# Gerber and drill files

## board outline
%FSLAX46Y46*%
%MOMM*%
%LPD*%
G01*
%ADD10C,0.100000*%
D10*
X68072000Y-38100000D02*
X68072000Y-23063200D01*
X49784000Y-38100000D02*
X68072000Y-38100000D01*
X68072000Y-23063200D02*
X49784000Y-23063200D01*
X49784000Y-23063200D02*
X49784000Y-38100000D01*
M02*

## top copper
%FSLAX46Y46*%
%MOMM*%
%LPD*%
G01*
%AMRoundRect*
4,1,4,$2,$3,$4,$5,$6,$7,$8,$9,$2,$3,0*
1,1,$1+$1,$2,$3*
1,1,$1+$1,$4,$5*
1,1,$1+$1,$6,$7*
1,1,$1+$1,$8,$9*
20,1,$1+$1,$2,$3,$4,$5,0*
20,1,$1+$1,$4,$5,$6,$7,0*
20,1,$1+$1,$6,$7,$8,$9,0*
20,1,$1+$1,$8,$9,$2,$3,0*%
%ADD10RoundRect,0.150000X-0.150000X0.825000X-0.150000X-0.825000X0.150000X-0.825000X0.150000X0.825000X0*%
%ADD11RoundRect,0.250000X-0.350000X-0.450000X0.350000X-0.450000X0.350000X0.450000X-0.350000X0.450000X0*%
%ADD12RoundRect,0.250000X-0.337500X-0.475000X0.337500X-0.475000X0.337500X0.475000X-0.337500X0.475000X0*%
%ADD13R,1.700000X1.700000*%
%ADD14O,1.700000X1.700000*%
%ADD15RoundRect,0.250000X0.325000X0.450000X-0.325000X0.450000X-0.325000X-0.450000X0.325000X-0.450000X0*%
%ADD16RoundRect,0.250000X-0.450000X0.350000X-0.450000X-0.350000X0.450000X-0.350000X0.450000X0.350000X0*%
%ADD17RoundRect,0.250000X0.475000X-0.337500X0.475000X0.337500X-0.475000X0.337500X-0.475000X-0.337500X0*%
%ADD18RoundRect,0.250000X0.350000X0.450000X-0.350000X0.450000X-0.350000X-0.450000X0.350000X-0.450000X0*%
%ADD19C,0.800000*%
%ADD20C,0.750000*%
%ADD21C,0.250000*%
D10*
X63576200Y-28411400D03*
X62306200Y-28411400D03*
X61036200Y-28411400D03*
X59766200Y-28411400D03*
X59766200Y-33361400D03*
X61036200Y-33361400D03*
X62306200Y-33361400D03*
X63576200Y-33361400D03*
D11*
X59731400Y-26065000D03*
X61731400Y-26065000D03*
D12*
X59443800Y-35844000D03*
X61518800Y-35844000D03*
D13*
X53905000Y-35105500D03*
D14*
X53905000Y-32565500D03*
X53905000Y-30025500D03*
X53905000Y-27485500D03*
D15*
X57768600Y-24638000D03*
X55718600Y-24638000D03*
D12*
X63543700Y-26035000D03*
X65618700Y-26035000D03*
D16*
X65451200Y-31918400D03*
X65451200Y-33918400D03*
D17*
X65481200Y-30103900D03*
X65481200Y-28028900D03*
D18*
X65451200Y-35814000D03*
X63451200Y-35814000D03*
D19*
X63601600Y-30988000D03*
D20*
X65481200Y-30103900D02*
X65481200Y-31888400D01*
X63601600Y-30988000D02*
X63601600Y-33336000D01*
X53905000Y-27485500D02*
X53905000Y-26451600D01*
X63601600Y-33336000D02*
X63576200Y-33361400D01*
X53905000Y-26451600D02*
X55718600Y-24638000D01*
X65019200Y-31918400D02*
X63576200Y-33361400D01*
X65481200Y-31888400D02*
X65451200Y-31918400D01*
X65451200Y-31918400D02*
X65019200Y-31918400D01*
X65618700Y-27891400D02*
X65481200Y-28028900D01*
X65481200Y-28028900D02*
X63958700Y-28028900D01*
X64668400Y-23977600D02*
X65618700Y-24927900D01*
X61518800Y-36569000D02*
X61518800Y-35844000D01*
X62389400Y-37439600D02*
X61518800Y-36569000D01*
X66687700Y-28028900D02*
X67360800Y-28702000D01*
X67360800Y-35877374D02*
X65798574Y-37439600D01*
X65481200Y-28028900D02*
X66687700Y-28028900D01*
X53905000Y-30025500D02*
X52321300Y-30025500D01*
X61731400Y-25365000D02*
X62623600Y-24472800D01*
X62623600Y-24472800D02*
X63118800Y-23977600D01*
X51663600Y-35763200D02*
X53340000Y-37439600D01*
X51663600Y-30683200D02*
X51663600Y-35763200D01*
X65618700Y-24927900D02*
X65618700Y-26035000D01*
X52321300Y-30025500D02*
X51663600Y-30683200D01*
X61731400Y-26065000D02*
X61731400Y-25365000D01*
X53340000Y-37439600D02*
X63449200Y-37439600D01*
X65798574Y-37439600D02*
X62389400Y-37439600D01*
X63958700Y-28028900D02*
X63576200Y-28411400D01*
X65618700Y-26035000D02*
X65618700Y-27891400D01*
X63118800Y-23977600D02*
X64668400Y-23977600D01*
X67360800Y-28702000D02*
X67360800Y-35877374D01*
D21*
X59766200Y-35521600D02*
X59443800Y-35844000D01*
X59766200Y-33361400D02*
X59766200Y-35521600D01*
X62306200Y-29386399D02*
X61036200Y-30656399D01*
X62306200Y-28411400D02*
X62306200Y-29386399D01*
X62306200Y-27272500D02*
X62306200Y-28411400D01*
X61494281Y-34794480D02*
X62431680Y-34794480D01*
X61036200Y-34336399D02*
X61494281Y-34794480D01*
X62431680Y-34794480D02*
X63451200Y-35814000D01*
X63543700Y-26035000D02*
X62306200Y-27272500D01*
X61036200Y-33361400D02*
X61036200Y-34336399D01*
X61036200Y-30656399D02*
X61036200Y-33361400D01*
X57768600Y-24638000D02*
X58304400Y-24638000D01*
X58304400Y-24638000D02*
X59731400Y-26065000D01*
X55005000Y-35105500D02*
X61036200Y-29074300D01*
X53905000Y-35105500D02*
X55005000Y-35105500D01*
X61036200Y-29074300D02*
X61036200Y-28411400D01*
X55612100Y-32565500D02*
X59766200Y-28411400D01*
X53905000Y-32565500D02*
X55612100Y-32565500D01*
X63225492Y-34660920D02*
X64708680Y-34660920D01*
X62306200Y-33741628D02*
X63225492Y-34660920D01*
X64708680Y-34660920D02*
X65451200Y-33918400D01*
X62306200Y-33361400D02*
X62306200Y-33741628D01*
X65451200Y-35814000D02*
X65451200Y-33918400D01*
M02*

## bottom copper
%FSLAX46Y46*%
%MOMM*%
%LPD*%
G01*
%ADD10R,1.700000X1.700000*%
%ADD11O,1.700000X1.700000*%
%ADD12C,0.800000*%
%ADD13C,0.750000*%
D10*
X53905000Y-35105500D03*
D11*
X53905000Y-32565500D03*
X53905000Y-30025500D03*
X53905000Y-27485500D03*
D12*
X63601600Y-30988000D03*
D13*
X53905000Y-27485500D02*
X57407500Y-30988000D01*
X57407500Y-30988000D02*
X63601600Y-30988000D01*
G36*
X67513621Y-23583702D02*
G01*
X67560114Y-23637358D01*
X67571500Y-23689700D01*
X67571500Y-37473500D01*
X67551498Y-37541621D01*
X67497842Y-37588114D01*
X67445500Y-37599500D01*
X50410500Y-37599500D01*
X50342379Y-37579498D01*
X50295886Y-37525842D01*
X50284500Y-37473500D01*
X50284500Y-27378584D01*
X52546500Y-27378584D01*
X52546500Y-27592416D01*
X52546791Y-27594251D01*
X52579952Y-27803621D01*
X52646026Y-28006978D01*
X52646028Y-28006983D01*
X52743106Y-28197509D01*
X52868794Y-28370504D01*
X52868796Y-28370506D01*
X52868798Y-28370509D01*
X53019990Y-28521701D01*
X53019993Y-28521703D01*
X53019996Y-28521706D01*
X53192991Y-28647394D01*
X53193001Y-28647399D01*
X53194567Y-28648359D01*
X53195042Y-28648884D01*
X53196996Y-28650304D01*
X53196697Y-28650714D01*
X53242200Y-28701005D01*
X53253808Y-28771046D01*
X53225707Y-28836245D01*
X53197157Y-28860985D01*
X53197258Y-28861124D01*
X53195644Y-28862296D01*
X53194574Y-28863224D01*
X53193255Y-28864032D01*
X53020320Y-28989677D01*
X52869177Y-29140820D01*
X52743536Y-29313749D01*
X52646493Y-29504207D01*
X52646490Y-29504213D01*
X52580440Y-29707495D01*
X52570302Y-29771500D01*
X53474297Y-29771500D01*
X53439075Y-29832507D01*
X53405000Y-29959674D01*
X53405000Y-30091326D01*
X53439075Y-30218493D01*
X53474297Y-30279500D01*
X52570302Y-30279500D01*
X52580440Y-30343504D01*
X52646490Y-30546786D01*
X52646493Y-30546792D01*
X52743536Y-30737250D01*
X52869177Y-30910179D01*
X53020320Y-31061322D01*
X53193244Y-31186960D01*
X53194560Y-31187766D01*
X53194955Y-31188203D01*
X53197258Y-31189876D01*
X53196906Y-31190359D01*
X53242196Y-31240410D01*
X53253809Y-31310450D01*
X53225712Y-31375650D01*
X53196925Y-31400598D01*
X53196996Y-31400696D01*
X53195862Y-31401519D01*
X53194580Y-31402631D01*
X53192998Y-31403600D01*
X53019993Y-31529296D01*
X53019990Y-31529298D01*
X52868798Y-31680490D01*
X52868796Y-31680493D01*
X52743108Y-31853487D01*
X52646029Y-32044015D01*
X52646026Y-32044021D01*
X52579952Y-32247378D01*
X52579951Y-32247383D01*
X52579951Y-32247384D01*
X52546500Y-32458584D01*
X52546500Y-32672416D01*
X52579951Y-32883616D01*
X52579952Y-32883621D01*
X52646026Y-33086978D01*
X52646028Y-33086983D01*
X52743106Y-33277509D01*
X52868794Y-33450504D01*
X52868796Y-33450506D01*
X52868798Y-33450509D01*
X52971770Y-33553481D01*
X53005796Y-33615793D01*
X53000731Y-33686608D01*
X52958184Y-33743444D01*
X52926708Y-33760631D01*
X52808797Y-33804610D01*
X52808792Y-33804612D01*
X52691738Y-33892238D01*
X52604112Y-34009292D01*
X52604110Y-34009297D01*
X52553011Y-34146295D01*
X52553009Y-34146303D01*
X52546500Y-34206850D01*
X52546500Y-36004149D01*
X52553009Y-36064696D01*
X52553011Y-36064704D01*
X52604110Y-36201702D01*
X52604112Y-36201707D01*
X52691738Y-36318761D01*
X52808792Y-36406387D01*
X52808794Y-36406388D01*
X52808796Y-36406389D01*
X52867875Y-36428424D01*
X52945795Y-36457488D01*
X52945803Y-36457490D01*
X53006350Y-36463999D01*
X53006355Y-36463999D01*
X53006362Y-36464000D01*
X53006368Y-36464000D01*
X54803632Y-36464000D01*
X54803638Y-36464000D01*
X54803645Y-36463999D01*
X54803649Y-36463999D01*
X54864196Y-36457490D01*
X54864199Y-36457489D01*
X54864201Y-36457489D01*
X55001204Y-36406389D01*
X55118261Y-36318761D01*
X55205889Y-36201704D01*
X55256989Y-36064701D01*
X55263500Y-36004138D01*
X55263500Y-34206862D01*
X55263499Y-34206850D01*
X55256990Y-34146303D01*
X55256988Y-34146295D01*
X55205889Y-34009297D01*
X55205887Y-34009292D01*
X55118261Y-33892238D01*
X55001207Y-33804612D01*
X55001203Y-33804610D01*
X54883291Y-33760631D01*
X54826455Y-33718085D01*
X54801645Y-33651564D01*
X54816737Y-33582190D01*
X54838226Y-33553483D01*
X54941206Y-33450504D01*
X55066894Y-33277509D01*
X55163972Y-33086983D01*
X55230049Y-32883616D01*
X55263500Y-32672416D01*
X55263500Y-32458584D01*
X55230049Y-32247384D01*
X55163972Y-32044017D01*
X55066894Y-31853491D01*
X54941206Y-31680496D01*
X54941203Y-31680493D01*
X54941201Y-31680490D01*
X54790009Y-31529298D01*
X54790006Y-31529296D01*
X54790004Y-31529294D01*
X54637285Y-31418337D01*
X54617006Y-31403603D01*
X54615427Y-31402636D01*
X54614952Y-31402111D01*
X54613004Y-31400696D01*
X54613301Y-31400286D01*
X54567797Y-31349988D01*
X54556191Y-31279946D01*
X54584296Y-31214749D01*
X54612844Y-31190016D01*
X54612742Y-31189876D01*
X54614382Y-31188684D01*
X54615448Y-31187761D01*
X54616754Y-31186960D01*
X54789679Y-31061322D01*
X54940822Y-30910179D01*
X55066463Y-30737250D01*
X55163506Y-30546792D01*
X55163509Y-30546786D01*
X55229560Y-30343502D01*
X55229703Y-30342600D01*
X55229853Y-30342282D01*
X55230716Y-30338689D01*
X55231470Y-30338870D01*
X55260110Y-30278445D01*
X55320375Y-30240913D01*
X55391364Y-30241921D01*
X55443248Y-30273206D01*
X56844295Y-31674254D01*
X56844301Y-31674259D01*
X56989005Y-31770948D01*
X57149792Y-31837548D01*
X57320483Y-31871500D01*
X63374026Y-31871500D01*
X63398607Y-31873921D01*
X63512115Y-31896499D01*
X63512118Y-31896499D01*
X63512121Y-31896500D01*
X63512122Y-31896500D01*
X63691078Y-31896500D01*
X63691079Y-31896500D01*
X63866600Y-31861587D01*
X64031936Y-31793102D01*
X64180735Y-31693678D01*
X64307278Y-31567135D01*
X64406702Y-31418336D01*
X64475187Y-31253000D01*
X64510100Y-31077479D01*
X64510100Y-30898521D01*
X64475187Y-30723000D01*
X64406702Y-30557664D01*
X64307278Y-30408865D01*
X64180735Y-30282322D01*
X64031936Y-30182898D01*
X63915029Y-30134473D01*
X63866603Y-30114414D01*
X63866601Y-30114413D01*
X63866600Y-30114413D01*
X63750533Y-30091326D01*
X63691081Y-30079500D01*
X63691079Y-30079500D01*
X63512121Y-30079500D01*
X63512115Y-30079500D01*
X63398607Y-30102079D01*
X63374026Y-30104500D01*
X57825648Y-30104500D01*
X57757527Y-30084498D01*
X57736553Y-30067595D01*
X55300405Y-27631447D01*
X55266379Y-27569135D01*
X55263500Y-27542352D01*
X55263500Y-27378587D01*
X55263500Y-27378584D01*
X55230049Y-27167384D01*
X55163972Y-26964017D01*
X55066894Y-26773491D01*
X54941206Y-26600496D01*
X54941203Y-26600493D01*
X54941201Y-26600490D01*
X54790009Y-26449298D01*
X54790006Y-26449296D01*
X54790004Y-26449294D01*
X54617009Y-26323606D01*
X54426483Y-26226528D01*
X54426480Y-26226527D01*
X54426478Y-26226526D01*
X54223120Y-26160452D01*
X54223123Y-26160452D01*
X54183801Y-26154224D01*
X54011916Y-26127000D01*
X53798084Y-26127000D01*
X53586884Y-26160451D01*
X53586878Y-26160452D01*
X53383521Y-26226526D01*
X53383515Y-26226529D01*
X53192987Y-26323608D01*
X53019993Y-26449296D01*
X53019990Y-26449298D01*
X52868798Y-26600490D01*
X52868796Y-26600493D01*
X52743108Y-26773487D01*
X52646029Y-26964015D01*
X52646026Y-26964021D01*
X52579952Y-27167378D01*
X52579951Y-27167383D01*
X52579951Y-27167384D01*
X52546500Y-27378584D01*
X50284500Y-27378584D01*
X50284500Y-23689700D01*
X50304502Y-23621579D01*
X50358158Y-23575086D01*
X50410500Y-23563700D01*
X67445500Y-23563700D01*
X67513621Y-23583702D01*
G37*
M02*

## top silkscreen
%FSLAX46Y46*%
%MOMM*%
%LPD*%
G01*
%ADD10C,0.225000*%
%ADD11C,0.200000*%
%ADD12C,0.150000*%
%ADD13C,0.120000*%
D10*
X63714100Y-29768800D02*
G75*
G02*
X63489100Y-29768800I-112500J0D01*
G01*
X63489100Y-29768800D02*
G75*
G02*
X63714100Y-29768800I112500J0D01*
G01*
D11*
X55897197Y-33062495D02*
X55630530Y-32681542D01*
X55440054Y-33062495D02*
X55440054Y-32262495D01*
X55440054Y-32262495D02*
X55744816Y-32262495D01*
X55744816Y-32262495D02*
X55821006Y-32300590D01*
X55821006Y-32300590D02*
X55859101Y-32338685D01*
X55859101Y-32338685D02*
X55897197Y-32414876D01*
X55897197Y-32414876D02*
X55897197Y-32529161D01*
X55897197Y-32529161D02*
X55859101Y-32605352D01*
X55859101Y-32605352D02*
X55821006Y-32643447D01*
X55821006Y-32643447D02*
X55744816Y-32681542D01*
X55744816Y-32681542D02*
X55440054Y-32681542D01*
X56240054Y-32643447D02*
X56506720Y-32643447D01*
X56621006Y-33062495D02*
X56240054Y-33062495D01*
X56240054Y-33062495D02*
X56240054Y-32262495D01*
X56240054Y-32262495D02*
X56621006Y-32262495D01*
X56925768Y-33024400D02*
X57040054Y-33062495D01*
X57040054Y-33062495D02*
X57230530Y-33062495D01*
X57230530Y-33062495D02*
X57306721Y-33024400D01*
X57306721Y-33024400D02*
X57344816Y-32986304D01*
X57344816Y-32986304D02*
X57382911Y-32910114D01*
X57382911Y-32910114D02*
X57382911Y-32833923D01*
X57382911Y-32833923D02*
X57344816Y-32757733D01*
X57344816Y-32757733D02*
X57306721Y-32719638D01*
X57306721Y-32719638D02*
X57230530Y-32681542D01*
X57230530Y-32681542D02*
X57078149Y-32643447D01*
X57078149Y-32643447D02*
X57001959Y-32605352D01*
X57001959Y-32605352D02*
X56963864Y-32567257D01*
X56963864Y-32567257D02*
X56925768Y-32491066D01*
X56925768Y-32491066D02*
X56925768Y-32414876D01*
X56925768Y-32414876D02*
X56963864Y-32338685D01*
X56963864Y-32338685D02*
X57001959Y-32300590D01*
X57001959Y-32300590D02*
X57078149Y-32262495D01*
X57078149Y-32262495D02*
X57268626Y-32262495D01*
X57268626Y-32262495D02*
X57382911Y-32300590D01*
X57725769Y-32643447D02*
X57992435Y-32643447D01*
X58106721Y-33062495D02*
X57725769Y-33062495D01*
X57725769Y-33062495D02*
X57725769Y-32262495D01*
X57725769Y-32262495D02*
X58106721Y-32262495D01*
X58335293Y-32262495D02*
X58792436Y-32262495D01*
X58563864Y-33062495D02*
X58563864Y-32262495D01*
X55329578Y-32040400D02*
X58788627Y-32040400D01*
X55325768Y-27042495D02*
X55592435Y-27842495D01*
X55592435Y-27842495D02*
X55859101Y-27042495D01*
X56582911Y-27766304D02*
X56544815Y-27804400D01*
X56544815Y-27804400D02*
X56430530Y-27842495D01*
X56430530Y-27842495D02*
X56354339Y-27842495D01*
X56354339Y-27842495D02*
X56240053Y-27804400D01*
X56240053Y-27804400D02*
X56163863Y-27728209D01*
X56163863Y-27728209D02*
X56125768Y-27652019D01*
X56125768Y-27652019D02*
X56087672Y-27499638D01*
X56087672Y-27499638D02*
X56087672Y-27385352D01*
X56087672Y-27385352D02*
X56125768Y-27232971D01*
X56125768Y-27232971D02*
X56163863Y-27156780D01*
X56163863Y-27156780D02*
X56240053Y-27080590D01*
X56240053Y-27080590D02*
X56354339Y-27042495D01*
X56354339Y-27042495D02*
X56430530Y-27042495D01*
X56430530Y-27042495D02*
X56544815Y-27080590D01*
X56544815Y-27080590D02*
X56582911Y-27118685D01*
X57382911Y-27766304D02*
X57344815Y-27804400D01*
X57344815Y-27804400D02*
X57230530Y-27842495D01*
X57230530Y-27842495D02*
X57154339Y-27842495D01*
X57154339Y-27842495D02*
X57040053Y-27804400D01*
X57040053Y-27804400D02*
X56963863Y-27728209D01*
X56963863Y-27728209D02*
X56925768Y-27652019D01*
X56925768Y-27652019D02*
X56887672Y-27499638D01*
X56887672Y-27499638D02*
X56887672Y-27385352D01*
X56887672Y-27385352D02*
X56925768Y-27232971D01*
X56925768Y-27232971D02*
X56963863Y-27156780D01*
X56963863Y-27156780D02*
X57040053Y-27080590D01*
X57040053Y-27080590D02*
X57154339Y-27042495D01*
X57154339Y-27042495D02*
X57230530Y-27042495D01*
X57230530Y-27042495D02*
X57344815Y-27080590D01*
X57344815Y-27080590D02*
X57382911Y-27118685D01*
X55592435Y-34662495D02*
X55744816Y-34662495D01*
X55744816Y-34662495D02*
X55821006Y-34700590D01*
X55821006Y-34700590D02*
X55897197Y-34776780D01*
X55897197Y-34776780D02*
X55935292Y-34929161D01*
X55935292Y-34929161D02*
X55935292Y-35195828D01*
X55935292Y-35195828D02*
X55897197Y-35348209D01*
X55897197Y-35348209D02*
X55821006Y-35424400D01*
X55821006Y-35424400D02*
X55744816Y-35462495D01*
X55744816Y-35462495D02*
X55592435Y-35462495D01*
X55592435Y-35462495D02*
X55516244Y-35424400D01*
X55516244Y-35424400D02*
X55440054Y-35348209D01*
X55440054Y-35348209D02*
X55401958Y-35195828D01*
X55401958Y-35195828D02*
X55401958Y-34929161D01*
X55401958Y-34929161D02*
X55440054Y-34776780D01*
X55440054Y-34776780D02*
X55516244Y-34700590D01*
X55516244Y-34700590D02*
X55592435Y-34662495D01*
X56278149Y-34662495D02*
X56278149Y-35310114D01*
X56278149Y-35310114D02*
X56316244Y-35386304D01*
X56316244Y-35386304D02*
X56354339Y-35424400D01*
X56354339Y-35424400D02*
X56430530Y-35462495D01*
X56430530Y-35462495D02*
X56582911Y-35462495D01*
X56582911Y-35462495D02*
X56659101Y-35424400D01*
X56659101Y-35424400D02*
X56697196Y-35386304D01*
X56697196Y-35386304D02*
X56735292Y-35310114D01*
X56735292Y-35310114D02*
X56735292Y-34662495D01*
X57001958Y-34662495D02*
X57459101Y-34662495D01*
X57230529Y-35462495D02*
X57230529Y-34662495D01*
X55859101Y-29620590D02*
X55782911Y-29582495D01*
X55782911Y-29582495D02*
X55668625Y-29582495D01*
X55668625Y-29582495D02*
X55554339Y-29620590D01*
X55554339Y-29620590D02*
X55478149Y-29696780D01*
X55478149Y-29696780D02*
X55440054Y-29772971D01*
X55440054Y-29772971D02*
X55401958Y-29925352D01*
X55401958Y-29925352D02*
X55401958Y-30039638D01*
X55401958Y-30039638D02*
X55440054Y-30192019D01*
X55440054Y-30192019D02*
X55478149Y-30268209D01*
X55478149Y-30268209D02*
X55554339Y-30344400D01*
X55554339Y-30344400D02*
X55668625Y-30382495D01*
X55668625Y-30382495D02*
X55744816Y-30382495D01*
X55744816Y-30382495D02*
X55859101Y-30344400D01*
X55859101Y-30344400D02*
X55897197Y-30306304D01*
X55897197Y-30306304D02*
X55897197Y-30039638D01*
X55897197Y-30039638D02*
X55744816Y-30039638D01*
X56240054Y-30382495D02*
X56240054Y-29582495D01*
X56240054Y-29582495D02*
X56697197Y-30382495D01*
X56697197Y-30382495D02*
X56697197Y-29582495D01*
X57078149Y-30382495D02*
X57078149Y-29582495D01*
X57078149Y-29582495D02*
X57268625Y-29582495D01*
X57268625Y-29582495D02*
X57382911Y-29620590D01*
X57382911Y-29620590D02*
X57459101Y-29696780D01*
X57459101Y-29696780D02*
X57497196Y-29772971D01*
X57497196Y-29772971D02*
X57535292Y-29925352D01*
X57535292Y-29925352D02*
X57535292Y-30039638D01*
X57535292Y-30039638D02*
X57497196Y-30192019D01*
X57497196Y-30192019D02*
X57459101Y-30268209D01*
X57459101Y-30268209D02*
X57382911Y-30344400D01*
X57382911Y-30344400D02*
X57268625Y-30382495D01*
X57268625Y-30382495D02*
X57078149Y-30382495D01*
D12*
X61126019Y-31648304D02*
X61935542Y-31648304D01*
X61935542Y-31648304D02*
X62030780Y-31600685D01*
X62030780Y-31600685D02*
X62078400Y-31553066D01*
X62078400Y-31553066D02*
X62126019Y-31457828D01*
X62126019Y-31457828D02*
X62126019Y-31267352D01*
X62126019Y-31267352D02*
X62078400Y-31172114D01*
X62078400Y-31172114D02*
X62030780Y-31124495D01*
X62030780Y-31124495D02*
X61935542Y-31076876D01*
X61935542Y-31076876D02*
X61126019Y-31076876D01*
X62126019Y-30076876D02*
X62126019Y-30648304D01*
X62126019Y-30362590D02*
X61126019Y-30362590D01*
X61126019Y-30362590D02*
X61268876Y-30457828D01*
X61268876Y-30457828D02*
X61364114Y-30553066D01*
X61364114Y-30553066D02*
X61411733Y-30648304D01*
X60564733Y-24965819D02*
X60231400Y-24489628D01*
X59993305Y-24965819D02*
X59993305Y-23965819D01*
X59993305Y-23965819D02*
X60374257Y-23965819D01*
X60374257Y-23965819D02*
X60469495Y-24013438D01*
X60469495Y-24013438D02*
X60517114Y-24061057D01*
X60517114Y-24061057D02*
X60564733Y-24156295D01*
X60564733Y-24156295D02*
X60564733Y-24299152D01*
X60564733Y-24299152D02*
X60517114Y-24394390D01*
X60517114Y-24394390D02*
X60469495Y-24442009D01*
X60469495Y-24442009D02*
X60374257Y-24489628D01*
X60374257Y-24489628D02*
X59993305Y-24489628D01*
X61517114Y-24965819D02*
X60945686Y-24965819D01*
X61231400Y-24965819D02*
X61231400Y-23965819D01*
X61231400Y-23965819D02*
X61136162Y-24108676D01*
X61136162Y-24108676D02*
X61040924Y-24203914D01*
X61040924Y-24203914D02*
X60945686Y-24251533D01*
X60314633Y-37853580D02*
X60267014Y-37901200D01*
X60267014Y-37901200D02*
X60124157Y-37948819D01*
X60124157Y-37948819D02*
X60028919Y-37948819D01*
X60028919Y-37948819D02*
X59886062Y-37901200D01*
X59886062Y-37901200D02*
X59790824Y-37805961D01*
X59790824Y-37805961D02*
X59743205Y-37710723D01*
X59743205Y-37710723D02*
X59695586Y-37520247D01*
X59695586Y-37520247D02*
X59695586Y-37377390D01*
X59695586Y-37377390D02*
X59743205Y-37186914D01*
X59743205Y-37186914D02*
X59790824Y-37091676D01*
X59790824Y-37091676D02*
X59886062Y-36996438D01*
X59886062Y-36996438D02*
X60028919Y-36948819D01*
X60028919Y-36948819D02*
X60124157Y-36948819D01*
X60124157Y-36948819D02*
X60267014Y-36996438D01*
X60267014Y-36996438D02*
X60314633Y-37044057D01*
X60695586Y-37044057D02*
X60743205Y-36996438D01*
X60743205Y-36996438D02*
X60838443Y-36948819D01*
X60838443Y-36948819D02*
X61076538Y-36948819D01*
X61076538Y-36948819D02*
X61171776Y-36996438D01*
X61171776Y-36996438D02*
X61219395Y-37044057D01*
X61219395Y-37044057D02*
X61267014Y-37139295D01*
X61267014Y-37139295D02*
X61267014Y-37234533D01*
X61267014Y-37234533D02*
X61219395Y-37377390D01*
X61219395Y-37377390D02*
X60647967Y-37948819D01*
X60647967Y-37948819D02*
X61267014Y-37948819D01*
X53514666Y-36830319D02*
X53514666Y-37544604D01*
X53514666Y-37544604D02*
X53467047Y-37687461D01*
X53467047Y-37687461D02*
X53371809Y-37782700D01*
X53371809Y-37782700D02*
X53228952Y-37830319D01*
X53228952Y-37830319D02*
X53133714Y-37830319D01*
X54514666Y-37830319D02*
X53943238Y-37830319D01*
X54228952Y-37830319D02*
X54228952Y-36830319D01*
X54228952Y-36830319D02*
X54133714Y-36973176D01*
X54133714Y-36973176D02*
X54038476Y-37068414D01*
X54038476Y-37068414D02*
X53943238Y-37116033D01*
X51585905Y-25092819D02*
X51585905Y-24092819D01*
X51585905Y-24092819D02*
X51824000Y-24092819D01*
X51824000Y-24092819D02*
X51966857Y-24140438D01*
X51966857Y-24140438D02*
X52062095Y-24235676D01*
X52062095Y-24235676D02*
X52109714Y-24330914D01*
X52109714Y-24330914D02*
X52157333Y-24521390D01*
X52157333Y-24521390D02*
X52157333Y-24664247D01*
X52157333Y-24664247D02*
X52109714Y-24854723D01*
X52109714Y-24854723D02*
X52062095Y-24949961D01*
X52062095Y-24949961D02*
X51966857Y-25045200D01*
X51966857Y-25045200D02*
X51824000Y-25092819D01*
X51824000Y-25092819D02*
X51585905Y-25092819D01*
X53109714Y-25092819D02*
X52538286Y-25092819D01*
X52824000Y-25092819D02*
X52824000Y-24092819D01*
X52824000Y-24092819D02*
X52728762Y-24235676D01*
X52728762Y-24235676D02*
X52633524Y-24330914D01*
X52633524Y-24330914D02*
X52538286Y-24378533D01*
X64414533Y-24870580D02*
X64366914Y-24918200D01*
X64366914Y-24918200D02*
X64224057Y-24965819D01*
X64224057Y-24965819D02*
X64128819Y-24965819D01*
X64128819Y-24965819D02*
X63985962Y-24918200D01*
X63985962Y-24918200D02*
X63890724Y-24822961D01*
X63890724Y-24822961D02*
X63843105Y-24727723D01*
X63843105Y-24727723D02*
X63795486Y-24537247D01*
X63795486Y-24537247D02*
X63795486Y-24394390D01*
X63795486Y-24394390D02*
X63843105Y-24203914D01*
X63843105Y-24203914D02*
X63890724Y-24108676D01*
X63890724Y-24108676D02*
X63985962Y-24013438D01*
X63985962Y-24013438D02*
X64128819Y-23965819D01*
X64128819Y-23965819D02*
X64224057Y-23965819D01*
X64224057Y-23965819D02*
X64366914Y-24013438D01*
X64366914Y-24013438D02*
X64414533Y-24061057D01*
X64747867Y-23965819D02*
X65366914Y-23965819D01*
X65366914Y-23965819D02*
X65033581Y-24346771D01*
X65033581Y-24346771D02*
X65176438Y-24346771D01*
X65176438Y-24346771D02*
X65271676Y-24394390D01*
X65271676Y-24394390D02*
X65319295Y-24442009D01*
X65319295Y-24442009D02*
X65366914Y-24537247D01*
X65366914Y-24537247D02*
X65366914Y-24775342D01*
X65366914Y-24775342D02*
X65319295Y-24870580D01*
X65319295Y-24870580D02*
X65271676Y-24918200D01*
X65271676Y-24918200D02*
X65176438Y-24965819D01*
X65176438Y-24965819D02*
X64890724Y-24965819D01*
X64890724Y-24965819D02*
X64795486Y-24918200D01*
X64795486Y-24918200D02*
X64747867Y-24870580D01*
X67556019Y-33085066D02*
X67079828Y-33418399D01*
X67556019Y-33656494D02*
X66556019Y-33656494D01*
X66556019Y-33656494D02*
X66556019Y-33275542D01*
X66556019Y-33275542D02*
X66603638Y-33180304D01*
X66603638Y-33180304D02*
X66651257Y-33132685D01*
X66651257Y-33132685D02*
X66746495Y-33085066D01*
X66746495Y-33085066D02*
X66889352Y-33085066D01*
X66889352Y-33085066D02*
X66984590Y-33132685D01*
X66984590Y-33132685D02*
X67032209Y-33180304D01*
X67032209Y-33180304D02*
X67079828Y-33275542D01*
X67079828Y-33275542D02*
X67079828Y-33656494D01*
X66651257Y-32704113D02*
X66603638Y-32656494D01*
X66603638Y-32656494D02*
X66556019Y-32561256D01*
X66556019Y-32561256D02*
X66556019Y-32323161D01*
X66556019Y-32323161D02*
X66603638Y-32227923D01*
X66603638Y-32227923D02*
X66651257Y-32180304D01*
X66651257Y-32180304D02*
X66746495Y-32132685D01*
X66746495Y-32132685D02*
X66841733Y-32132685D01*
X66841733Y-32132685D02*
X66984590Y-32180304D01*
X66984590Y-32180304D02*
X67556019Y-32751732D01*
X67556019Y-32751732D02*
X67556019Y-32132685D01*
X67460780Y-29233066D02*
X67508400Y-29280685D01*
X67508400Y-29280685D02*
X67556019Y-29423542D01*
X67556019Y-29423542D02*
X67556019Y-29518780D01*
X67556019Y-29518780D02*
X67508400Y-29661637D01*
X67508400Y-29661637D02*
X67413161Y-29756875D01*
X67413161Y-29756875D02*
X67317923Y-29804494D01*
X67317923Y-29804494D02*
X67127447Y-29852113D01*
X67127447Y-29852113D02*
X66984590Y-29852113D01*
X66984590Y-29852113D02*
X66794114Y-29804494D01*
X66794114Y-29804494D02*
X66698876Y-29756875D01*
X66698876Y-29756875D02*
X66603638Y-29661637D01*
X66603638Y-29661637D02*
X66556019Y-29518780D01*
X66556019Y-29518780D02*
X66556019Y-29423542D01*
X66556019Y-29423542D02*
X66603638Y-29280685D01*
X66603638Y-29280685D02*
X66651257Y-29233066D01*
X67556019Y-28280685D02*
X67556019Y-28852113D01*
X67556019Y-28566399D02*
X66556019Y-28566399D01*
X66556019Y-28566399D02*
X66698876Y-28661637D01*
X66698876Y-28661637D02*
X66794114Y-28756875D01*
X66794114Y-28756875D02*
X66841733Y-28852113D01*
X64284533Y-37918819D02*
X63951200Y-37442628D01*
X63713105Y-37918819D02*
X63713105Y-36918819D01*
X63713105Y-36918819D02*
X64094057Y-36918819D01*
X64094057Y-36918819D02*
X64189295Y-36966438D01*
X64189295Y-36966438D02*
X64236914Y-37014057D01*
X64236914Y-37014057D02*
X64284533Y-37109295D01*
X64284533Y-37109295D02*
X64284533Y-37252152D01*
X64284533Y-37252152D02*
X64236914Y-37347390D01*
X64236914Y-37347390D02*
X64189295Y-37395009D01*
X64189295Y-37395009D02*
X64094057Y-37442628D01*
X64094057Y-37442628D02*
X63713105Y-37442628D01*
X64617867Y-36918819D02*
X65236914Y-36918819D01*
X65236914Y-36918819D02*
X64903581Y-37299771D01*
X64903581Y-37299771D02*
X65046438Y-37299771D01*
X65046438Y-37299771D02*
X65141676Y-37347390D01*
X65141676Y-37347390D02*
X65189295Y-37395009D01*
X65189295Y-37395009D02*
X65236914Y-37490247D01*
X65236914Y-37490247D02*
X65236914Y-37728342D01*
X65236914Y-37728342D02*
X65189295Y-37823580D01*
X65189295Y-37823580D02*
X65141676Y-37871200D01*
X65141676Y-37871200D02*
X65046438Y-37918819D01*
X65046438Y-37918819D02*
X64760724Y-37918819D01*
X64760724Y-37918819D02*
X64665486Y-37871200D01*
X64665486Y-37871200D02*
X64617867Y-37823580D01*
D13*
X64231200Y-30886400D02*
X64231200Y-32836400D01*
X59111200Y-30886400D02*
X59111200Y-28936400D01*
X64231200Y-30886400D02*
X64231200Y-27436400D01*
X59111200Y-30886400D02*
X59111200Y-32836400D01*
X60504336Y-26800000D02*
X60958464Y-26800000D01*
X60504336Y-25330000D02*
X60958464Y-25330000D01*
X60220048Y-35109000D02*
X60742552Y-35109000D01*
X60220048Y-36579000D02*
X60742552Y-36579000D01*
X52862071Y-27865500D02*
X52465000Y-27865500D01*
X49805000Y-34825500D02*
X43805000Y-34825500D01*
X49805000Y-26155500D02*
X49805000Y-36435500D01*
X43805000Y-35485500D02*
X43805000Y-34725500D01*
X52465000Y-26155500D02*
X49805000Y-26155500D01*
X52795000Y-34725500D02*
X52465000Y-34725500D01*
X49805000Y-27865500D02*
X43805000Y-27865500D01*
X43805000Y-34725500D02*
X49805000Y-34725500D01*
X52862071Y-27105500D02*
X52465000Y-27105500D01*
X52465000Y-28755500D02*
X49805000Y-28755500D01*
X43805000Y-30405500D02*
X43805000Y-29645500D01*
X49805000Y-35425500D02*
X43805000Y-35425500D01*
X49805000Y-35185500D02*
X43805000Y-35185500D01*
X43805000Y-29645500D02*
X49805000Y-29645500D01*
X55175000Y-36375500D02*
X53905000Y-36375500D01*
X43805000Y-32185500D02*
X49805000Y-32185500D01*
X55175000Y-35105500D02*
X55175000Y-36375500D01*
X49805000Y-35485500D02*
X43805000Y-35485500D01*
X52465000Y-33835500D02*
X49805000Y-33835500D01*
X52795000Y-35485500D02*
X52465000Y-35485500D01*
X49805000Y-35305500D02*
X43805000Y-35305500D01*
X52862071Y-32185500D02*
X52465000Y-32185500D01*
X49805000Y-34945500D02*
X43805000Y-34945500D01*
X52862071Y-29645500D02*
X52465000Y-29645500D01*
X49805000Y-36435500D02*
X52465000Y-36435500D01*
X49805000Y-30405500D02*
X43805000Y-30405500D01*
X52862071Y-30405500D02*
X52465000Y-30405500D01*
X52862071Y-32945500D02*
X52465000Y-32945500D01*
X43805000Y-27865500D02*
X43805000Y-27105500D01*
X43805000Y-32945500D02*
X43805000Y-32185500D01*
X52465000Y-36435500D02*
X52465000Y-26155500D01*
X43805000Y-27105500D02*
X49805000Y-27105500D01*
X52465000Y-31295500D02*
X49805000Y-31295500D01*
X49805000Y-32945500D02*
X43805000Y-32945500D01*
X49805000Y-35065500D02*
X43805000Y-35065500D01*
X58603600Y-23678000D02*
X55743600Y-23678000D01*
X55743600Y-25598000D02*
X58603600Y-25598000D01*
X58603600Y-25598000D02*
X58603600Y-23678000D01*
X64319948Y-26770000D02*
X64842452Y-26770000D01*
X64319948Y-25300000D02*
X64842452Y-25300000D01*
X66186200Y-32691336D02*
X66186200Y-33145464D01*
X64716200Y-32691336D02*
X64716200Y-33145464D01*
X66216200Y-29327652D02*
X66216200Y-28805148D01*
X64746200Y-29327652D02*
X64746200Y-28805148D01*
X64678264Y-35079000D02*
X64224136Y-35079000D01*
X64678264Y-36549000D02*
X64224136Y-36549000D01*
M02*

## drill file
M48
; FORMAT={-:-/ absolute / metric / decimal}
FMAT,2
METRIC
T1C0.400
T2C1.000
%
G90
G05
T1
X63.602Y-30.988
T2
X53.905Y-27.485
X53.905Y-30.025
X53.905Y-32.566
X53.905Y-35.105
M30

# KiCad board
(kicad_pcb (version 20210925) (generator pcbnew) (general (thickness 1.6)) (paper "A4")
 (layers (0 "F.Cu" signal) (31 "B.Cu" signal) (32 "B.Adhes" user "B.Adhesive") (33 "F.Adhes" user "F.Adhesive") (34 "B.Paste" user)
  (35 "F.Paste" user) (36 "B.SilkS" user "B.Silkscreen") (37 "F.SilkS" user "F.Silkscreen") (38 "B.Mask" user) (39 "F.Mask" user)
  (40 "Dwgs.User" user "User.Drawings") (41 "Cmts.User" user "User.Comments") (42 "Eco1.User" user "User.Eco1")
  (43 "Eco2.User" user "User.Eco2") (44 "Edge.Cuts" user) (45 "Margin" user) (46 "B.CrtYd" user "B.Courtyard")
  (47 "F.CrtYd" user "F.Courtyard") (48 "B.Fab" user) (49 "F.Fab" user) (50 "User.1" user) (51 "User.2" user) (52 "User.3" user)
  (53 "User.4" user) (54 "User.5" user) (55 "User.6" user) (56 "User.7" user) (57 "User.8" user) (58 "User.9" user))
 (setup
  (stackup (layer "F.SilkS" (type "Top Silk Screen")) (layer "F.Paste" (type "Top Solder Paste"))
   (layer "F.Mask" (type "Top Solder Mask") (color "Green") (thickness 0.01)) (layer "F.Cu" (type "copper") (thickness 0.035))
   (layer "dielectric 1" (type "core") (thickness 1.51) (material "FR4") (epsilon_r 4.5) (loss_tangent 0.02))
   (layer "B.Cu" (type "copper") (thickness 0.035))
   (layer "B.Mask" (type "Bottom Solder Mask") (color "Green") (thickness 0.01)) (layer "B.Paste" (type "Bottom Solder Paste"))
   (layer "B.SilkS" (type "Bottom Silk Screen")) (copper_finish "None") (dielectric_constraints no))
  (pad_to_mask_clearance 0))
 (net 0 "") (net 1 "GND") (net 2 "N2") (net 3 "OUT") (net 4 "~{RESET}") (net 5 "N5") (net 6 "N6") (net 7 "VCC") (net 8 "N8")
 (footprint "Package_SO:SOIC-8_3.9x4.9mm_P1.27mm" (layer "F.Cu") (at 61.6712 30.8864 -90)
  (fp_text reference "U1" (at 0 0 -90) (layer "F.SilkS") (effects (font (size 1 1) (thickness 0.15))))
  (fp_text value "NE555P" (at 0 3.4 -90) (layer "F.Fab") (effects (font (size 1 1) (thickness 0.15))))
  (fp_line (start 0 -2.56) (end 1.95 -2.56) (layer "F.SilkS") (width 0.12))
  (fp_line (start 0 2.56) (end -1.95 2.56) (layer "F.SilkS") (width 0.12))
  (fp_line (start 0 -2.56) (end -3.45 -2.56) (layer "F.SilkS") (width 0.12))
  (fp_line (start 0 2.56) (end 1.95 2.56) (layer "F.SilkS") (width 0.12))
  (pad "1" smd roundrect locked (at -2.475 -1.905 270) (size 1.95 0.6) (layers "F.Cu" "F.Paste" "F.Mask") (roundrect_rratio 0.25)
   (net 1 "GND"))
  (pad "2" smd roundrect locked (at -2.475 -0.635 270) (size 1.95 0.6) (layers "F.Cu" "F.Paste" "F.Mask") (roundrect_rratio 0.25)
   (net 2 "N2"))
  (pad "3" smd roundrect locked (at -2.475 0.635 270) (size 1.95 0.6) (layers "F.Cu" "F.Paste" "F.Mask") (roundrect_rratio 0.25)
   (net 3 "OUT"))
  (pad "4" smd roundrect locked (at -2.475 1.905 270) (size 1.95 0.6) (layers "F.Cu" "F.Paste" "F.Mask") (roundrect_rratio 0.25)
   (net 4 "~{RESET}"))
  (pad "5" smd roundrect locked (at 2.475 1.905 270) (size 1.95 0.6) (layers "F.Cu" "F.Paste" "F.Mask") (roundrect_rratio 0.25) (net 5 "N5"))
  (pad "6" smd roundrect locked (at 2.475 0.635 270) (size 1.95 0.6) (layers "F.Cu" "F.Paste" "F.Mask") (roundrect_rratio 0.25) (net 2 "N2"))
  (pad "7" smd roundrect locked (at 2.475 -0.635 270) (size 1.95 0.6) (layers "F.Cu" "F.Paste" "F.Mask") (roundrect_rratio 0.25)
   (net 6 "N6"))
  (pad "8" smd roundrect locked (at 2.475 -1.905 270) (size 1.95 0.6) (layers "F.Cu" "F.Paste" "F.Mask") (roundrect_rratio 0.25)
   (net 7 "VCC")))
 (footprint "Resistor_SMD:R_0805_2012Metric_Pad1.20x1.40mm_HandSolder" (layer "F.Cu") (at 60.7314 26.065)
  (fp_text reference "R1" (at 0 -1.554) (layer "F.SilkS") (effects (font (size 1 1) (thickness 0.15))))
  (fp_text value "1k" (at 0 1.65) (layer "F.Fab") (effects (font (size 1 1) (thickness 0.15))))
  (fp_line (start -0.227064 0.735) (end 0.227064 0.735) (layer "F.SilkS") (width 0.12))
  (fp_line (start -0.227064 -0.735) (end 0.227064 -0.735) (layer "F.SilkS") (width 0.12))
  (pad "1" smd roundrect locked (at -1 0) (size 1.2 1.4) (layers "F.Cu" "F.Paste" "F.Mask") (roundrect_rratio 0.208333) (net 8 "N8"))
  (pad "2" smd roundrect locked (at 1 0) (size 1.2 1.4) (layers "F.Cu" "F.Paste" "F.Mask") (roundrect_rratio 0.208333) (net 1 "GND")))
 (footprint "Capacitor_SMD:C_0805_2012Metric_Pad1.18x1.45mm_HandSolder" (layer "F.Cu") (at 60.4813 35.844)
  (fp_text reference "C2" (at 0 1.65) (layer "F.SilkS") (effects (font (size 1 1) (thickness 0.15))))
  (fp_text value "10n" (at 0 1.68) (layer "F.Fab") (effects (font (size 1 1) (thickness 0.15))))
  (fp_line (start -0.261252 -0.735) (end 0.261252 -0.735) (layer "F.SilkS") (width 0.12))
  (fp_line (start -0.261252 0.735) (end 0.261252 0.735) (layer "F.SilkS") (width 0.12))
  (pad "1" smd roundrect locked (at -1.0375 0) (size 1.175 1.45) (layers "F.Cu" "F.Paste" "F.Mask") (roundrect_rratio 0.212766) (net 5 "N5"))
  (pad "2" smd roundrect locked (at 1.0375 0) (size 1.175 1.45) (layers "F.Cu" "F.Paste" "F.Mask") (roundrect_rratio 0.212766) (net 1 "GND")))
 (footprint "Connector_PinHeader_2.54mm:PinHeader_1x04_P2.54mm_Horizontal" (layer "F.Cu") (at 53.905 35.1055 180)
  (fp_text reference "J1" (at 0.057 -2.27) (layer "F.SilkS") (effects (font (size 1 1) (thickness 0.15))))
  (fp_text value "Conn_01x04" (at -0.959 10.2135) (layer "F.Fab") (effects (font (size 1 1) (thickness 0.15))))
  (fp_line (start 1.042929 7.24) (end 1.44 7.24) (layer "F.SilkS") (width 0.12))
  (fp_line (start 4.1 0.28) (end 10.1 0.28) (layer "F.SilkS") (width 0.12))
  (fp_line (start 4.1 8.95) (end 4.1 -1.33) (layer "F.SilkS") (width 0.12))
  (fp_line (start 10.1 -0.38) (end 10.1 0.38) (layer "F.SilkS") (width 0.12))
  (fp_line (start 1.44 8.95) (end 4.1 8.95) (layer "F.SilkS") (width 0.12))
  (fp_line (start 1.11 0.38) (end 1.44 0.38) (layer "F.SilkS") (width 0.12))
  (fp_line (start 4.1 7.24) (end 10.1 7.24) (layer "F.SilkS") (width 0.12))
  (fp_line (start 10.1 0.38) (end 4.1 0.38) (layer "F.SilkS") (width 0.12))
  (fp_line (start 1.042929 8) (end 1.44 8) (layer "F.SilkS") (width 0.12))
  (fp_line (start 1.44 6.35) (end 4.1 6.35) (layer "F.SilkS") (width 0.12))
  (fp_line (start 10.1 4.7) (end 10.1 5.46) (layer "F.SilkS") (width 0.12))
  (fp_line (start 4.1 -0.32) (end 10.1 -0.32) (layer "F.SilkS") (width 0.12))
  (fp_line (start 4.1 -0.08) (end 10.1 -0.08) (layer "F.SilkS") (width 0.12))
  (fp_line (start 10.1 5.46) (end 4.1 5.46) (layer "F.SilkS") (width 0.12))
  (fp_line (start -1.27 -1.27) (end 0 -1.27) (layer "F.SilkS") (width 0.12))
  (fp_line (start 10.1 2.92) (end 4.1 2.92) (layer "F.SilkS") (width 0.12))
  (fp_line (start -1.27 0) (end -1.27 -1.27) (layer "F.SilkS") (width 0.12))
  (fp_line (start 4.1 -0.38) (end 10.1 -0.38) (layer "F.SilkS") (width 0.12))
  (fp_line (start 1.44 1.27) (end 4.1 1.27) (layer "F.SilkS") (width 0.12))
  (fp_line (start 1.11 -0.38) (end 1.44 -0.38) (layer "F.SilkS") (width 0.12))
  (fp_line (start 4.1 -0.2) (end 10.1 -0.2) (layer "F.SilkS") (width 0.12))
  (fp_line (start 1.042929 2.92) (end 1.44 2.92) (layer "F.SilkS") (width 0.12))
  (fp_line (start 4.1 0.16) (end 10.1 0.16) (layer "F.SilkS") (width 0.12))
  (fp_line (start 1.042929 5.46) (end 1.44 5.46) (layer "F.SilkS") (width 0.12))
  (fp_line (start 4.1 -1.33) (end 1.44 -1.33) (layer "F.SilkS") (width 0.12))
  (fp_line (start 4.1 4.7) (end 10.1 4.7) (layer "F.SilkS") (width 0.12))
  (fp_line (start 1.042929 4.7) (end 1.44 4.7) (layer "F.SilkS") (width 0.12))
  (fp_line (start 1.042929 2.16) (end 1.44 2.16) (layer "F.SilkS") (width 0.12))
  (fp_line (start 10.1 7.24) (end 10.1 8) (layer "F.SilkS") (width 0.12))
  (fp_line (start 10.1 2.16) (end 10.1 2.92) (layer "F.SilkS") (width 0.12))
  (fp_line (start 1.44 -1.33) (end 1.44 8.95) (layer "F.SilkS") (width 0.12))
  (fp_line (start 10.1 8) (end 4.1 8) (layer "F.SilkS") (width 0.12))
  (fp_line (start 1.44 3.81) (end 4.1 3.81) (layer "F.SilkS") (width 0.12))
  (fp_line (start 4.1 2.16) (end 10.1 2.16) (layer "F.SilkS") (width 0.12))
  (fp_line (start 4.1 0.04) (end 10.1 0.04) (layer "F.SilkS") (width 0.12))
  (pad "1" thru_hole rect locked (at 0 0 180) (size 1.7 1.7) (drill 1) (layers *.Cu *.Mask) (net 3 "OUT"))
  (pad "2" thru_hole oval locked (at 0 2.54 180) (size 1.7 1.7) (drill 1) (layers *.Cu *.Mask) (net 4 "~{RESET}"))
  (pad "3" thru_hole oval locked (at 0 5.08 180) (size 1.7 1.7) (drill 1) (layers *.Cu *.Mask) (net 1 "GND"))
  (pad "4" thru_hole oval locked (at 0 7.62 180) (size 1.7 1.7) (drill 1) (layers *.Cu *.Mask) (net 7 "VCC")))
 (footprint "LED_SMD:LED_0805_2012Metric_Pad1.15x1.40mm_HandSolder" (layer "F.Cu") (at 56.7436 24.638 180)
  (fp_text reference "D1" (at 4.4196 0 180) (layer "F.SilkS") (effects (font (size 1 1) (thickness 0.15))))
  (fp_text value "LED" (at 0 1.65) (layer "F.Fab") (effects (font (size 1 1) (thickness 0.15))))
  (fp_line (start -1.86 0.96) (end 1 0.96) (layer "F.SilkS") (width 0.12))
  (fp_line (start 1 -0.96) (end -1.86 -0.96) (layer "F.SilkS") (width 0.12))
  (fp_line (start -1.86 -0.96) (end -1.86 0.96) (layer "F.SilkS") (width 0.12))
  (pad "1" smd roundrect locked (at -1.025 0 180) (size 1.15 1.4) (layers "F.Cu" "F.Paste" "F.Mask") (roundrect_rratio 0.217391)
   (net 8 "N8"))
  (pad "2" smd roundrect locked (at 1.025 0 180) (size 1.15 1.4) (layers "F.Cu" "F.Paste" "F.Mask") (roundrect_rratio 0.217391)
   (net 7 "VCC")))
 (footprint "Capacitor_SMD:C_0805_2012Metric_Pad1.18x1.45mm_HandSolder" (layer "F.Cu") (at 64.5812 26.035)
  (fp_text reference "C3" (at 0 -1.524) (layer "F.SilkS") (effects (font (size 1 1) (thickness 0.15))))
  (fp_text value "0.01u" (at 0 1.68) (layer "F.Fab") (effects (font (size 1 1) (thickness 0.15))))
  (fp_line (start -0.261252 0.735) (end 0.261252 0.735) (layer "F.SilkS") (width 0.12))
  (fp_line (start -0.261252 -0.735) (end 0.261252 -0.735) (layer "F.SilkS") (width 0.12))
  (pad "1" smd roundrect locked (at -1.0375 0) (size 1.175 1.45) (layers "F.Cu" "F.Paste" "F.Mask") (roundrect_rratio 0.212766) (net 2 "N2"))
  (pad "2" smd roundrect locked (at 1.0375 0) (size 1.175 1.45) (layers "F.Cu" "F.Paste" "F.Mask") (roundrect_rratio 0.212766) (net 1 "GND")))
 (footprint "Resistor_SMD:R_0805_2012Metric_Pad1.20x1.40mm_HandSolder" (layer "F.Cu") (at 65.4512 32.9184 -90)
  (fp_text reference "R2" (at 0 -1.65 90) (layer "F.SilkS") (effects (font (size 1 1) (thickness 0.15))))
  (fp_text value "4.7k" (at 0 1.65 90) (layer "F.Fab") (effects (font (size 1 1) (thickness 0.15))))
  (fp_line (start -0.227064 -0.735) (end 0.227064 -0.735) (layer "F.SilkS") (width 0.12))
  (fp_line (start -0.227064 0.735) (end 0.227064 0.735) (layer "F.SilkS") (width 0.12))
  (pad "1" smd roundrect locked (at -1 0 270) (size 1.2 1.4) (layers "F.Cu" "F.Paste" "F.Mask") (roundrect_rratio 0.208333) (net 7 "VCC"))
  (pad "2" smd roundrect locked (at 1 0 270) (size 1.2 1.4) (layers "F.Cu" "F.Paste" "F.Mask") (roundrect_rratio 0.208333) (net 6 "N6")))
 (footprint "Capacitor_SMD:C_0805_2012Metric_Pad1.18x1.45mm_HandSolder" (layer "F.Cu") (at 65.4812 29.0664 90)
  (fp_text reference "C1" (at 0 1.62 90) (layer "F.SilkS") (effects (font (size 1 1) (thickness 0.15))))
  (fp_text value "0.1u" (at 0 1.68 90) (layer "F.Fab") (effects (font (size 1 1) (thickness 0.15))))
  (fp_line (start -0.261252 0.735) (end 0.261252 0.735) (layer "F.SilkS") (width 0.12))
  (fp_line (start -0.261252 -0.735) (end 0.261252 -0.735) (layer "F.SilkS") (width 0.12))
  (pad "1" smd roundrect locked (at -1.0375 0 90) (size 1.175 1.45) (layers "F.Cu" "F.Paste" "F.Mask") (roundrect_rratio 0.212766)
   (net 7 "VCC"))
  (pad "2" smd roundrect locked (at 1.0375 0 90) (size 1.175 1.45) (layers "F.Cu" "F.Paste" "F.Mask") (roundrect_rratio 0.212766)
   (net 1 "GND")))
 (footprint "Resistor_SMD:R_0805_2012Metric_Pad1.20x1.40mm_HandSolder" (layer "F.Cu") (at 64.4512 35.814 180)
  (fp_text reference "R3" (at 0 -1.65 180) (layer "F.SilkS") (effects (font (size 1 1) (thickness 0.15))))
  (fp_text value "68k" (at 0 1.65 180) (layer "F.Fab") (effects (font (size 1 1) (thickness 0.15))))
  (fp_line (start -0.227064 0.735) (end 0.227064 0.735) (layer "F.SilkS") (width 0.12))
  (fp_line (start -0.227064 -0.735) (end 0.227064 -0.735) (layer "F.SilkS") (width 0.12))
  (pad "1" smd roundrect locked (at -1 0 180) (size 1.2 1.4) (layers "F.Cu" "F.Paste" "F.Mask") (roundrect_rratio 0.208333) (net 6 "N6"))
  (pad "2" smd roundrect locked (at 1 0 180) (size 1.2 1.4) (layers "F.Cu" "F.Paste" "F.Mask") (roundrect_rratio 0.208333) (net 2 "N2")))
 (gr_circle (center 63.6016 29.7688) (end 63.7516 29.7688) (layer "F.SilkS") (width 0.15) (fill solid))
 (gr_line (start 68.072 38.1) (end 68.072 23.0632) (layer "Edge.Cuts") (width 0.1))
 (gr_line (start 49.784 38.1) (end 68.072 38.1) (layer "Edge.Cuts") (width 0.1))
 (gr_line (start 68.072 23.0632) (end 49.784 23.0632) (layer "Edge.Cuts") (width 0.1))
 (gr_line (start 49.784 23.0632) (end 49.784 38.1) (layer "Edge.Cuts") (width 0.1))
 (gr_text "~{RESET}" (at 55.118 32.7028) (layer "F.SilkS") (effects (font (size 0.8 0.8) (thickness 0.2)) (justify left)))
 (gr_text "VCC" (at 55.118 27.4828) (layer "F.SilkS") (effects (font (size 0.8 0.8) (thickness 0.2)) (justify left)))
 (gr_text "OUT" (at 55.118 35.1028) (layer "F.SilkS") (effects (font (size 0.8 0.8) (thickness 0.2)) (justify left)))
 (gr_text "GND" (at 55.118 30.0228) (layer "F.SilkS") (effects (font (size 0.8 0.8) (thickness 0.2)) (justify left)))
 (segment (start 65.4812 30.1039) (end 65.4812 31.8884) (width 0.75) (layer "F.Cu") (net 7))
 (segment (start 63.6016 30.988) (end 63.6016 33.336) (width 0.75) (layer "F.Cu") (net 7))
 (segment (start 53.905 27.4855) (end 53.905 26.4516) (width 0.75) (layer "F.Cu") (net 7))
 (segment (start 63.6016 33.336) (end 63.5762 33.3614) (width 0.75) (layer "F.Cu") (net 7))
 (segment (start 53.905 26.4516) (end 55.7186 24.638) (width 0.75) (layer "F.Cu") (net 7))
 (segment (start 65.0192 31.9184) (end 63.5762 33.3614) (width 0.75) (layer "F.Cu") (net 7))
 (segment (start 65.4812 31.8884) (end 65.4512 31.9184) (width 0.75) (layer "F.Cu") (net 7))
 (segment (start 65.4512 31.9184) (end 65.0192 31.9184) (width 0.75) (layer "F.Cu") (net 7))
 (via (at 63.6016 30.988) (size 0.8) (drill 0.4) (layers "F.Cu" "B.Cu") (free) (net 7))
 (segment (start 53.905 27.4855) (end 57.4075 30.988) (width 0.75) (layer "B.Cu") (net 7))
 (segment (start 57.4075 30.988) (end 63.6016 30.988) (width 0.75) (layer "B.Cu") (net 7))
 (segment (start 65.6187 27.8914) (end 65.4812 28.0289) (width 0.75) (layer "F.Cu") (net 1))
 (segment (start 65.4812 28.0289) (end 63.9587 28.0289) (width 0.75) (layer "F.Cu") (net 1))
 (segment (start 64.6684 23.9776) (end 65.6187 24.9279) (width 0.75) (layer "F.Cu") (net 1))
 (segment (start 61.5188 36.569) (end 61.5188 35.844) (width 0.75) (layer "F.Cu") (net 1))
 (segment (start 62.3894 37.4396) (end 61.5188 36.569) (width 0.75) (layer "F.Cu") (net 1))
 (segment (start 66.6877 28.0289) (end 67.3608 28.702) (width 0.75) (layer "F.Cu") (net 1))
 (segment (start 67.3608 35.877374) (end 65.798574 37.4396) (width 0.75) (layer "F.Cu") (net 1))
 (segment (start 65.4812 28.0289) (end 66.6877 28.0289) (width 0.75) (layer "F.Cu") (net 1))
 (segment (start 53.905 30.0255) (end 52.3213 30.0255) (width 0.75) (layer "F.Cu") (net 1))
 (segment (start 61.7314 25.365) (end 62.6236 24.4728) (width 0.75) (layer "F.Cu") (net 1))
 (segment (start 62.6236 24.4728) (end 63.1188 23.9776) (width 0.75) (layer "F.Cu") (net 1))
 (segment (start 51.6636 35.7632) (end 53.34 37.4396) (width 0.75) (layer "F.Cu") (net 1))
 (segment (start 51.6636 30.6832) (end 51.6636 35.7632) (width 0.75) (layer "F.Cu") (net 1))
 (segment (start 65.6187 24.9279) (end 65.6187 26.035) (width 0.75) (layer "F.Cu") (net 1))
 (segment (start 52.3213 30.0255) (end 51.6636 30.6832) (width 0.75) (layer "F.Cu") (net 1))
 (segment (start 61.7314 26.065) (end 61.7314 25.365) (width 0.75) (layer "F.Cu") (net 1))
 (segment (start 53.34 37.4396) (end 63.4492 37.4396) (width 0.75) (layer "F.Cu") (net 1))
 (segment (start 65.798574 37.4396) (end 62.3894 37.4396) (width 0.75) (layer "F.Cu") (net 1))
 (segment (start 63.9587 28.0289) (end 63.5762 28.4114) (width 0.75) (layer "F.Cu") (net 1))
 (segment (start 65.6187 26.035) (end 65.6187 27.8914) (width 0.75) (layer "F.Cu") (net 1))
 (segment (start 63.1188 23.9776) (end 64.6684 23.9776) (width 0.75) (layer "F.Cu") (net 1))
 (segment (start 67.3608 28.702) (end 67.3608 35.877374) (width 0.75) (layer "F.Cu") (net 1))
 (segment (start 59.7662 35.5216) (end 59.4438 35.844) (width 0.25) (layer "F.Cu") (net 5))
 (segment (start 59.7662 33.3614) (end 59.7662 35.5216) (width 0.25) (layer "F.Cu") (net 5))
 (segment (start 62.3062 29.386399) (end 61.0362 30.656399) (width 0.25) (layer "F.Cu") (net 2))
 (segment (start 62.3062 28.4114) (end 62.3062 29.386399) (width 0.25) (layer "F.Cu") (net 2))
 (segment (start 62.3062 27.2725) (end 62.3062 28.4114) (width 0.25) (layer "F.Cu") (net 2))
 (segment (start 61.494281 34.79448) (end 62.43168 34.79448) (width 0.25) (layer "F.Cu") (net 2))
 (segment (start 61.0362 34.336399) (end 61.494281 34.79448) (width 0.25) (layer "F.Cu") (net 2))
 (segment (start 62.43168 34.79448) (end 63.4512 35.814) (width 0.25) (layer "F.Cu") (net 2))
 (segment (start 63.5437 26.035) (end 62.3062 27.2725) (width 0.25) (layer "F.Cu") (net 2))
 (segment (start 61.0362 33.3614) (end 61.0362 34.336399) (width 0.25) (layer "F.Cu") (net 2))
 (segment (start 61.0362 30.656399) (end 61.0362 33.3614) (width 0.25) (layer "F.Cu") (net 2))
 (segment (start 57.7686 24.638) (end 58.3044 24.638) (width 0.25) (layer "F.Cu") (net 8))
 (segment (start 58.3044 24.638) (end 59.7314 26.065) (width 0.25) (layer "F.Cu") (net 8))
 (segment (start 55.005 35.1055) (end 61.0362 29.0743) (width 0.25) (layer "F.Cu") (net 3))
 (segment (start 53.905 35.1055) (end 55.005 35.1055) (width 0.25) (layer "F.Cu") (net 3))
 (segment (start 61.0362 29.0743) (end 61.0362 28.4114) (width 0.25) (layer "F.Cu") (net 3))
 (segment (start 55.6121 32.5655) (end 59.7662 28.4114) (width 0.25) (layer "F.Cu") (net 4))
 (segment (start 53.905 32.5655) (end 55.6121 32.5655) (width 0.25) (layer "F.Cu") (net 4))
 (segment (start 63.225492 34.66092) (end 64.70868 34.66092) (width 0.25) (layer "F.Cu") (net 6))
 (segment (start 62.3062 33.741628) (end 63.225492 34.66092) (width 0.25) (layer "F.Cu") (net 6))
 (segment (start 64.70868 34.66092) (end 65.4512 33.9184) (width 0.25) (layer "F.Cu") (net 6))
 (segment (start 62.3062 33.3614) (end 62.3062 33.741628) (width 0.25) (layer "F.Cu") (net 6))
 (segment (start 65.4512 35.814) (end 65.4512 33.9184) (width 0.25) (layer "F.Cu") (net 6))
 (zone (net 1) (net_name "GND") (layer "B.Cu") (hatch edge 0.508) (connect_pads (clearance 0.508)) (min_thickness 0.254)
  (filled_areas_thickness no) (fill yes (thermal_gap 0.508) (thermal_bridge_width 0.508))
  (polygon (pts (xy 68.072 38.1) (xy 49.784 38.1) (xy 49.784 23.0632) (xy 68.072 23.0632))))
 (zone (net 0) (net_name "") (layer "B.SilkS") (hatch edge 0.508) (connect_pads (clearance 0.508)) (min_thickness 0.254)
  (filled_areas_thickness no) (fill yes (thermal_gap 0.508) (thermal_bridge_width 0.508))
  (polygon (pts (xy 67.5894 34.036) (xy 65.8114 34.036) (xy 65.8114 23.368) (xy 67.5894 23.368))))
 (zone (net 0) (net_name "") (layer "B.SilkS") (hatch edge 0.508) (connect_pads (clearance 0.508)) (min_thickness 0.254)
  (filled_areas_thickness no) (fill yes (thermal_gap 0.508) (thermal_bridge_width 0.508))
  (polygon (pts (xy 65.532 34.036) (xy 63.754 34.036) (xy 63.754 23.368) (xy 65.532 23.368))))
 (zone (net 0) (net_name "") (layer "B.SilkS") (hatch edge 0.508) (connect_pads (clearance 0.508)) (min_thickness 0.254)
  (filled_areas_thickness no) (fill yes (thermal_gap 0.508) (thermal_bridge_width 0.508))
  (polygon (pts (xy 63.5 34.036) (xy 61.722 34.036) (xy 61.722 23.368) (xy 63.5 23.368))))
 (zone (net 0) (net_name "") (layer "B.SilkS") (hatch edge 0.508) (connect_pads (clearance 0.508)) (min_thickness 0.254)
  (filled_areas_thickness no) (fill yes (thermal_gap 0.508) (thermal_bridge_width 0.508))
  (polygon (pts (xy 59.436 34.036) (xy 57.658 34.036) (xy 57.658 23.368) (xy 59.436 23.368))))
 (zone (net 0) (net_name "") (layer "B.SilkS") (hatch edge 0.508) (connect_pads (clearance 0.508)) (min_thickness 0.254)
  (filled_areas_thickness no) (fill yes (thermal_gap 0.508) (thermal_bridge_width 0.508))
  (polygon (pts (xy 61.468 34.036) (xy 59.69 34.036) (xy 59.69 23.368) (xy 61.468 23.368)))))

